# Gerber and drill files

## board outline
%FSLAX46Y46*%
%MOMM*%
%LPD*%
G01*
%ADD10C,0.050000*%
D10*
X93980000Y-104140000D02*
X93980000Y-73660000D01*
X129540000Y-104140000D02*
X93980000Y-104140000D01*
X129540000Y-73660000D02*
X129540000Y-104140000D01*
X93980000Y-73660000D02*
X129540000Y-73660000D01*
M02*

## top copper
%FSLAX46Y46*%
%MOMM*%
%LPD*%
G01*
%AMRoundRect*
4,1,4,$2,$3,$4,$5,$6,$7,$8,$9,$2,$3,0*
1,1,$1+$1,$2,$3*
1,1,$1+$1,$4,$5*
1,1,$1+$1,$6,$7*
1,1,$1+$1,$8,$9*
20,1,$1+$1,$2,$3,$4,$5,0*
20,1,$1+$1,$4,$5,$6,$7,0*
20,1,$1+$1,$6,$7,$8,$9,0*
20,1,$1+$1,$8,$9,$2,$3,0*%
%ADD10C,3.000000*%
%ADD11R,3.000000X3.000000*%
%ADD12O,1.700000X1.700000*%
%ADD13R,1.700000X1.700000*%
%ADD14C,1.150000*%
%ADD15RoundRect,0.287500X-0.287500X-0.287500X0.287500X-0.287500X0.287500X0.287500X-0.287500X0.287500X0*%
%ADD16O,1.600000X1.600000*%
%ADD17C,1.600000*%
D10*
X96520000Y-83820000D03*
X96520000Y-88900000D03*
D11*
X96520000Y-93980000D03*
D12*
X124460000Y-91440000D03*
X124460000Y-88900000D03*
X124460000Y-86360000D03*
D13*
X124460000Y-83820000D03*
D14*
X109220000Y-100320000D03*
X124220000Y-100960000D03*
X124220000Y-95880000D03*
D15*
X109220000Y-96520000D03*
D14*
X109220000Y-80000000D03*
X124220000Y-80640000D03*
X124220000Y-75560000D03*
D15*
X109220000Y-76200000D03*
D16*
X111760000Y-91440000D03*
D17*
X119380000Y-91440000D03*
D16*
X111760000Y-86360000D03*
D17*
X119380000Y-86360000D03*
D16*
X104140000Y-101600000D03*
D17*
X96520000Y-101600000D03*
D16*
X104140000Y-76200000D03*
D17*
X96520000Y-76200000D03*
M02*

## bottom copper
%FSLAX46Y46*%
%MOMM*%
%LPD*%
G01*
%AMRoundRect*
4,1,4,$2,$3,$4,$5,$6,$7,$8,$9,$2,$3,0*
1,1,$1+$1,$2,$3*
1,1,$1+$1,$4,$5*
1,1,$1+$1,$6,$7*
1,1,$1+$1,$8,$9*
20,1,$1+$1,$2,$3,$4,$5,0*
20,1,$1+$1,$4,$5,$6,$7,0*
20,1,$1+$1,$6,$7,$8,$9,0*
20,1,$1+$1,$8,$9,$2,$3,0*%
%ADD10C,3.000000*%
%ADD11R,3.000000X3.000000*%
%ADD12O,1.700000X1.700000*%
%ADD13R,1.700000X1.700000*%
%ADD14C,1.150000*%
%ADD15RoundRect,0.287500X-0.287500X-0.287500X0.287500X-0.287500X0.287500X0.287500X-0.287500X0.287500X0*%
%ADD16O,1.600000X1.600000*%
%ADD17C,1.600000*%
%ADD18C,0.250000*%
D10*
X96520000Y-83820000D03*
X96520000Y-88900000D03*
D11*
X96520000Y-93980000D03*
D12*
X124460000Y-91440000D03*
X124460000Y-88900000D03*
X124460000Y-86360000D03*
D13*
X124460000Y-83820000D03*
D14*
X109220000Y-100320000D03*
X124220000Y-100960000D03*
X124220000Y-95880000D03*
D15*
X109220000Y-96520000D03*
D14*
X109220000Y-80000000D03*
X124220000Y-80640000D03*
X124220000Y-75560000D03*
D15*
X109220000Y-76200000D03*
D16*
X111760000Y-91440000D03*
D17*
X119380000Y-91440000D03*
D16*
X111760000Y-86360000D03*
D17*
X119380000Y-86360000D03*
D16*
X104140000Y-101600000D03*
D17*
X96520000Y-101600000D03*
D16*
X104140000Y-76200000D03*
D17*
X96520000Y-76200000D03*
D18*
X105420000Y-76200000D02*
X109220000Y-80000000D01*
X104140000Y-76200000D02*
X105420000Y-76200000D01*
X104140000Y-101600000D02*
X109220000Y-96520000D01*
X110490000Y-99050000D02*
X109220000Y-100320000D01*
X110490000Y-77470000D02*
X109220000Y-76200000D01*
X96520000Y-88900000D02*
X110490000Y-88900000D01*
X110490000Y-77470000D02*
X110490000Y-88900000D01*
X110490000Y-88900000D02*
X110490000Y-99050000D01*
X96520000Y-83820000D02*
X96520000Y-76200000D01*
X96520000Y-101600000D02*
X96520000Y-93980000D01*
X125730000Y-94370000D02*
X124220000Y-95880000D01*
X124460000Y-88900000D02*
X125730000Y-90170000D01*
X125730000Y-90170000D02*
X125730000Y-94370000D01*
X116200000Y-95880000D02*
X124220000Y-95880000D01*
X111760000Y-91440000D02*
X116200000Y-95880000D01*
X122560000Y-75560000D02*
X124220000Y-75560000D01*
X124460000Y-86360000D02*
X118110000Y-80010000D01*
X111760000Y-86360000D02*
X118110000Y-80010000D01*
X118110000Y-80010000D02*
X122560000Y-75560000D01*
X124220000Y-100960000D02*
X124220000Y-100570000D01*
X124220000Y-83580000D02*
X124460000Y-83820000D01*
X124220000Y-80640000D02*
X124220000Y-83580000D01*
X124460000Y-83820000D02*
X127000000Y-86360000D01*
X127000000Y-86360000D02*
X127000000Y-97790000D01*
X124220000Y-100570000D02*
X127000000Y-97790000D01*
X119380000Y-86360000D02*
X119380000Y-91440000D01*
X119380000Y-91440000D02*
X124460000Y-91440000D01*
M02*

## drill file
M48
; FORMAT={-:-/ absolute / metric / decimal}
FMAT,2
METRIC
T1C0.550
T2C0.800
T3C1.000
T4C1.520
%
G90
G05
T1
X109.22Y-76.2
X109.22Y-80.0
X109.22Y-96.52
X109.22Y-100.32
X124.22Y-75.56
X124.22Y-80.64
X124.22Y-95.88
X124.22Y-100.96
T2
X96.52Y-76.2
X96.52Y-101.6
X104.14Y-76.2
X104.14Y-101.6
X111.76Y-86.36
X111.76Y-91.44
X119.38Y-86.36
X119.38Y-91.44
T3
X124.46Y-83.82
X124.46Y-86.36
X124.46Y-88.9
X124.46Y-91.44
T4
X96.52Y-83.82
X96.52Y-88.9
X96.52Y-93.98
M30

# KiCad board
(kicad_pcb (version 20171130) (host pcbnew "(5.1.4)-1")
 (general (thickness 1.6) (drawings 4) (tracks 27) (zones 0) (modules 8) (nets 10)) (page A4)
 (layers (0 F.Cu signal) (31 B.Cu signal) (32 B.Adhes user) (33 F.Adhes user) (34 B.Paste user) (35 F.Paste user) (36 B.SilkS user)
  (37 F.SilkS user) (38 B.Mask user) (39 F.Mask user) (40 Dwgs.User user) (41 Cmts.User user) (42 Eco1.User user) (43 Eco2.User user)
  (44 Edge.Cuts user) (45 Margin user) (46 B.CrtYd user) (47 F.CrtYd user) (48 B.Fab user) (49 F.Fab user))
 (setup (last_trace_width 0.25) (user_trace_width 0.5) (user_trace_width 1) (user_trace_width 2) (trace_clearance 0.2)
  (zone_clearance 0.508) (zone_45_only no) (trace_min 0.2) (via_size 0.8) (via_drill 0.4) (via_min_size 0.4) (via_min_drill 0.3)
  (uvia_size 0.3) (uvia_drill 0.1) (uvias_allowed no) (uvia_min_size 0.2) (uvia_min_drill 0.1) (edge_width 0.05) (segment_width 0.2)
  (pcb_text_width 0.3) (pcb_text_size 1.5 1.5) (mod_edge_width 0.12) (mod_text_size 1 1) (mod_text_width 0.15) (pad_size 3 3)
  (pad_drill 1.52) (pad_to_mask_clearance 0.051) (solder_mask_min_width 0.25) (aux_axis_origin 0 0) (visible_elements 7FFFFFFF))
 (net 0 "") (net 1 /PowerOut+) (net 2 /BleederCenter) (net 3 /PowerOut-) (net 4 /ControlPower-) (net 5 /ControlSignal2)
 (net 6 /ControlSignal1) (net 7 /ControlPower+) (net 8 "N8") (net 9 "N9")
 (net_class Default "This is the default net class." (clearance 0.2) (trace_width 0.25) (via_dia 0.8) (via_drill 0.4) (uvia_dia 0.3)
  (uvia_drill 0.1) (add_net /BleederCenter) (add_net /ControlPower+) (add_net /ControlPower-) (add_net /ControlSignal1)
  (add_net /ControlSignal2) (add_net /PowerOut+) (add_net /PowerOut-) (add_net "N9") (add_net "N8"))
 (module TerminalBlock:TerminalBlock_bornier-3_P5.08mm (layer F.Cu) (at 96.52 93.98 90)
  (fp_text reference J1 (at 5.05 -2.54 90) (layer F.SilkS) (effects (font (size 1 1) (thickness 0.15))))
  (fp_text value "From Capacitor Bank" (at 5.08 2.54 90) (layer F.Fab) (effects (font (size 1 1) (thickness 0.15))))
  (pad 3 thru_hole circle (at 10.16 0 90) (size 3 3) (drill 1.52) (layers *.Cu *.Mask) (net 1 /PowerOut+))
  (pad 2 thru_hole circle (at 5.08 0 90) (size 3 3) (drill 1.52) (layers *.Cu *.Mask) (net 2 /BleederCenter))
  (pad 1 thru_hole rect (at 0 0 90) (size 3 3) (drill 1.52) (layers *.Cu *.Mask) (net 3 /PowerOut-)))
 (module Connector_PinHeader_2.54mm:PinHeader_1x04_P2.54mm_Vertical (layer F.Cu) (at 124.46 83.82)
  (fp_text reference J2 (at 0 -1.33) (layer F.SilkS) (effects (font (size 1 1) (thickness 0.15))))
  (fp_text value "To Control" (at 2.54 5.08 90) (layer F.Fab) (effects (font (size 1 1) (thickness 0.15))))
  (pad 4 thru_hole oval (at 0 7.62) (size 1.7 1.7) (drill 1) (layers *.Cu *.Mask) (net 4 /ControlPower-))
  (pad 3 thru_hole oval (at 0 5.08) (size 1.7 1.7) (drill 1) (layers *.Cu *.Mask) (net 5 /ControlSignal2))
  (pad 2 thru_hole oval (at 0 2.54) (size 1.7 1.7) (drill 1) (layers *.Cu *.Mask) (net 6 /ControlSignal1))
  (pad 1 thru_hole rect (at 0 0) (size 1.7 1.7) (drill 1) (layers *.Cu *.Mask) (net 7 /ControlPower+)))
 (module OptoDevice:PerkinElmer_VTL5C (layer F.Cu) (at 109.22 96.52)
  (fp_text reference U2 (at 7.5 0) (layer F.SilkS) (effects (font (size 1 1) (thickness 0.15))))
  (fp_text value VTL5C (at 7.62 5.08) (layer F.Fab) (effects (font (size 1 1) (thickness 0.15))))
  (pad 2 thru_hole circle (at 0 3.8) (size 1.15 1.15) (drill 0.55) (layers *.Cu *.Mask) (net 2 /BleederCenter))
  (pad 4 thru_hole circle (at 15 4.44) (size 1.15 1.15) (drill 0.55) (layers *.Cu *.Mask) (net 7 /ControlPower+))
  (pad 3 thru_hole circle (at 15 -0.64) (size 1.15 1.15) (drill 0.55) (layers *.Cu *.Mask) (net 5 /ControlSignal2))
  (pad 1 thru_hole roundrect (at 0 0) (size 1.15 1.15) (drill 0.55) (layers *.Cu *.Mask) (roundrect_rratio 0.25) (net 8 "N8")))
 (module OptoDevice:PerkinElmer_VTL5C (layer F.Cu) (at 109.22 76.2)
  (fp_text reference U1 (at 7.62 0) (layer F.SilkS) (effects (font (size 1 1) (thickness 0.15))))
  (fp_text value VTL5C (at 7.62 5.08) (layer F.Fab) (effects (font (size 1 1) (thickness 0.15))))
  (pad 2 thru_hole circle (at 0 3.8) (size 1.15 1.15) (drill 0.55) (layers *.Cu *.Mask) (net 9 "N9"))
  (pad 4 thru_hole circle (at 15 4.44) (size 1.15 1.15) (drill 0.55) (layers *.Cu *.Mask) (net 7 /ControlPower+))
  (pad 3 thru_hole circle (at 15 -0.64) (size 1.15 1.15) (drill 0.55) (layers *.Cu *.Mask) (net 6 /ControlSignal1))
  (pad 1 thru_hole roundrect (at 0 0) (size 1.15 1.15) (drill 0.55) (layers *.Cu *.Mask) (roundrect_rratio 0.25) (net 2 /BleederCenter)))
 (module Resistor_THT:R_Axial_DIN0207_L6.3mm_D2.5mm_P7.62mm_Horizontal (layer F.Cu) (at 119.38 91.44 180)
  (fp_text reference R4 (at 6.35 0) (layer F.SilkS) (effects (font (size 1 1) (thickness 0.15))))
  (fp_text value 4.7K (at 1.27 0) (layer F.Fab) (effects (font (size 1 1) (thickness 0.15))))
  (pad 2 thru_hole oval (at 7.62 0 180) (size 1.6 1.6) (drill 0.8) (layers *.Cu *.Mask) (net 5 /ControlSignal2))
  (pad 1 thru_hole circle (at 0 0 180) (size 1.6 1.6) (drill 0.8) (layers *.Cu *.Mask) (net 4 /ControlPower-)))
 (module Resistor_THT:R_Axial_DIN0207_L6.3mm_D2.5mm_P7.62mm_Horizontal (layer F.Cu) (at 119.38 86.36 180)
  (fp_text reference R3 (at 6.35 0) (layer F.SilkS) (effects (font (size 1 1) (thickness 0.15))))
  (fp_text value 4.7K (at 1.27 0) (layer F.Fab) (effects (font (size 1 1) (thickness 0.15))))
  (pad 2 thru_hole oval (at 7.62 0 180) (size 1.6 1.6) (drill 0.8) (layers *.Cu *.Mask) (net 6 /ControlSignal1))
  (pad 1 thru_hole circle (at 0 0 180) (size 1.6 1.6) (drill 0.8) (layers *.Cu *.Mask) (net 4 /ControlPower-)))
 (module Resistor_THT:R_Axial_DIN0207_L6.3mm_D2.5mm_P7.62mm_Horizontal (layer F.Cu) (at 96.52 101.6)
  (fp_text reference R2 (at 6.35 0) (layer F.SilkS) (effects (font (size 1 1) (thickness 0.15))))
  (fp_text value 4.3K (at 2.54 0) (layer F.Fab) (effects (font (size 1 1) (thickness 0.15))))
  (pad 2 thru_hole oval (at 7.62 0) (size 1.6 1.6) (drill 0.8) (layers *.Cu *.Mask) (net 8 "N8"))
  (pad 1 thru_hole circle (at 0 0) (size 1.6 1.6) (drill 0.8) (layers *.Cu *.Mask) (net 3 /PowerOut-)))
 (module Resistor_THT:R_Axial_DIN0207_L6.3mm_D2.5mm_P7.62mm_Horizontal (layer F.Cu) (at 96.52 76.2)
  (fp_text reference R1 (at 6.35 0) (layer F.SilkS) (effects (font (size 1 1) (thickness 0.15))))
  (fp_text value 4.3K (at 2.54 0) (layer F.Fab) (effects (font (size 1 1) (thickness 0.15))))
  (pad 2 thru_hole oval (at 7.62 0) (size 1.6 1.6) (drill 0.8) (layers *.Cu *.Mask) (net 9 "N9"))
  (pad 1 thru_hole circle (at 0 0) (size 1.6 1.6) (drill 0.8) (layers *.Cu *.Mask) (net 1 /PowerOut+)))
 (gr_line (start 93.98 104.14) (end 93.98 73.66) (layer Edge.Cuts) (width 0.05))
 (gr_line (start 129.54 104.14) (end 93.98 104.14) (layer Edge.Cuts) (width 0.05))
 (gr_line (start 129.54 73.66) (end 129.54 104.14) (layer Edge.Cuts) (width 0.05))
 (gr_line (start 93.98 73.66) (end 129.54 73.66) (layer Edge.Cuts) (width 0.05))
 (segment (start 105.42 76.2) (end 109.22 80) (width 0.25) (layer B.Cu) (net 9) (status 20))
 (segment (start 104.14 76.2) (end 105.42 76.2) (width 0.25) (layer B.Cu) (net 9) (status 10))
 (segment (start 104.14 101.6) (end 109.22 96.52) (width 0.25) (layer B.Cu) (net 8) (status 30))
 (segment (start 110.49 99.05) (end 109.22 100.32) (width 0.25) (layer B.Cu) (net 2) (status 20))
 (segment (start 110.49 77.47) (end 109.22 76.2) (width 0.25) (layer B.Cu) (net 2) (status 20))
 (segment (start 96.52 88.9) (end 110.49 88.9) (width 0.25) (layer B.Cu) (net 2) (status 10))
 (segment (start 110.49 77.47) (end 110.49 88.9) (width 0.25) (layer B.Cu) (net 2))
 (segment (start 110.49 88.9) (end 110.49 99.05) (width 0.25) (layer B.Cu) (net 2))
 (segment (start 96.52 83.82) (end 96.52 76.2) (width 0.25) (layer B.Cu) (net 1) (status 30))
 (segment (start 96.52 101.6) (end 96.52 93.98) (width 0.25) (layer B.Cu) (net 3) (status 30))
 (segment (start 125.73 94.37) (end 124.22 95.88) (width 0.25) (layer B.Cu) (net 5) (status 20))
 (segment (start 124.46 88.9) (end 125.73 90.17) (width 0.25) (layer B.Cu) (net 5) (status 10))
 (segment (start 125.73 90.17) (end 125.73 94.37) (width 0.25) (layer B.Cu) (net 5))
 (segment (start 116.2 95.88) (end 124.22 95.88) (width 0.25) (layer B.Cu) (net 5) (status 20))
 (segment (start 111.76 91.44) (end 116.2 95.88) (width 0.25) (layer B.Cu) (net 5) (status 10))
 (segment (start 122.56 75.56) (end 124.22 75.56) (width 0.25) (layer B.Cu) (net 6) (status 20))
 (segment (start 124.46 86.36) (end 118.11 80.01) (width 0.25) (layer B.Cu) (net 6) (status 10))
 (segment (start 111.76 86.36) (end 118.11 80.01) (width 0.25) (layer B.Cu) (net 6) (status 10))
 (segment (start 118.11 80.01) (end 122.56 75.56) (width 0.25) (layer B.Cu) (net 6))
 (segment (start 124.22 100.96) (end 124.22 100.57) (width 0.25) (layer B.Cu) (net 7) (status 30))
 (segment (start 124.22 83.58) (end 124.46 83.82) (width 0.25) (layer B.Cu) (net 7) (status 30))
 (segment (start 124.22 80.64) (end 124.22 83.58) (width 0.25) (layer B.Cu) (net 7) (status 30))
 (segment (start 124.46 83.82) (end 127 86.36) (width 0.25) (layer B.Cu) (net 7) (status 10))
 (segment (start 127 86.36) (end 127 97.79) (width 0.25) (layer B.Cu) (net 7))
 (segment (start 124.22 100.57) (end 127 97.79) (width 0.25) (layer B.Cu) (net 7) (status 10))
 (segment (start 119.38 86.36) (end 119.38 91.44) (width 0.25) (layer B.Cu) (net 4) (status 30))
 (segment (start 119.38 91.44) (end 124.46 91.44) (width 0.25) (layer B.Cu) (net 4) (status 30)))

